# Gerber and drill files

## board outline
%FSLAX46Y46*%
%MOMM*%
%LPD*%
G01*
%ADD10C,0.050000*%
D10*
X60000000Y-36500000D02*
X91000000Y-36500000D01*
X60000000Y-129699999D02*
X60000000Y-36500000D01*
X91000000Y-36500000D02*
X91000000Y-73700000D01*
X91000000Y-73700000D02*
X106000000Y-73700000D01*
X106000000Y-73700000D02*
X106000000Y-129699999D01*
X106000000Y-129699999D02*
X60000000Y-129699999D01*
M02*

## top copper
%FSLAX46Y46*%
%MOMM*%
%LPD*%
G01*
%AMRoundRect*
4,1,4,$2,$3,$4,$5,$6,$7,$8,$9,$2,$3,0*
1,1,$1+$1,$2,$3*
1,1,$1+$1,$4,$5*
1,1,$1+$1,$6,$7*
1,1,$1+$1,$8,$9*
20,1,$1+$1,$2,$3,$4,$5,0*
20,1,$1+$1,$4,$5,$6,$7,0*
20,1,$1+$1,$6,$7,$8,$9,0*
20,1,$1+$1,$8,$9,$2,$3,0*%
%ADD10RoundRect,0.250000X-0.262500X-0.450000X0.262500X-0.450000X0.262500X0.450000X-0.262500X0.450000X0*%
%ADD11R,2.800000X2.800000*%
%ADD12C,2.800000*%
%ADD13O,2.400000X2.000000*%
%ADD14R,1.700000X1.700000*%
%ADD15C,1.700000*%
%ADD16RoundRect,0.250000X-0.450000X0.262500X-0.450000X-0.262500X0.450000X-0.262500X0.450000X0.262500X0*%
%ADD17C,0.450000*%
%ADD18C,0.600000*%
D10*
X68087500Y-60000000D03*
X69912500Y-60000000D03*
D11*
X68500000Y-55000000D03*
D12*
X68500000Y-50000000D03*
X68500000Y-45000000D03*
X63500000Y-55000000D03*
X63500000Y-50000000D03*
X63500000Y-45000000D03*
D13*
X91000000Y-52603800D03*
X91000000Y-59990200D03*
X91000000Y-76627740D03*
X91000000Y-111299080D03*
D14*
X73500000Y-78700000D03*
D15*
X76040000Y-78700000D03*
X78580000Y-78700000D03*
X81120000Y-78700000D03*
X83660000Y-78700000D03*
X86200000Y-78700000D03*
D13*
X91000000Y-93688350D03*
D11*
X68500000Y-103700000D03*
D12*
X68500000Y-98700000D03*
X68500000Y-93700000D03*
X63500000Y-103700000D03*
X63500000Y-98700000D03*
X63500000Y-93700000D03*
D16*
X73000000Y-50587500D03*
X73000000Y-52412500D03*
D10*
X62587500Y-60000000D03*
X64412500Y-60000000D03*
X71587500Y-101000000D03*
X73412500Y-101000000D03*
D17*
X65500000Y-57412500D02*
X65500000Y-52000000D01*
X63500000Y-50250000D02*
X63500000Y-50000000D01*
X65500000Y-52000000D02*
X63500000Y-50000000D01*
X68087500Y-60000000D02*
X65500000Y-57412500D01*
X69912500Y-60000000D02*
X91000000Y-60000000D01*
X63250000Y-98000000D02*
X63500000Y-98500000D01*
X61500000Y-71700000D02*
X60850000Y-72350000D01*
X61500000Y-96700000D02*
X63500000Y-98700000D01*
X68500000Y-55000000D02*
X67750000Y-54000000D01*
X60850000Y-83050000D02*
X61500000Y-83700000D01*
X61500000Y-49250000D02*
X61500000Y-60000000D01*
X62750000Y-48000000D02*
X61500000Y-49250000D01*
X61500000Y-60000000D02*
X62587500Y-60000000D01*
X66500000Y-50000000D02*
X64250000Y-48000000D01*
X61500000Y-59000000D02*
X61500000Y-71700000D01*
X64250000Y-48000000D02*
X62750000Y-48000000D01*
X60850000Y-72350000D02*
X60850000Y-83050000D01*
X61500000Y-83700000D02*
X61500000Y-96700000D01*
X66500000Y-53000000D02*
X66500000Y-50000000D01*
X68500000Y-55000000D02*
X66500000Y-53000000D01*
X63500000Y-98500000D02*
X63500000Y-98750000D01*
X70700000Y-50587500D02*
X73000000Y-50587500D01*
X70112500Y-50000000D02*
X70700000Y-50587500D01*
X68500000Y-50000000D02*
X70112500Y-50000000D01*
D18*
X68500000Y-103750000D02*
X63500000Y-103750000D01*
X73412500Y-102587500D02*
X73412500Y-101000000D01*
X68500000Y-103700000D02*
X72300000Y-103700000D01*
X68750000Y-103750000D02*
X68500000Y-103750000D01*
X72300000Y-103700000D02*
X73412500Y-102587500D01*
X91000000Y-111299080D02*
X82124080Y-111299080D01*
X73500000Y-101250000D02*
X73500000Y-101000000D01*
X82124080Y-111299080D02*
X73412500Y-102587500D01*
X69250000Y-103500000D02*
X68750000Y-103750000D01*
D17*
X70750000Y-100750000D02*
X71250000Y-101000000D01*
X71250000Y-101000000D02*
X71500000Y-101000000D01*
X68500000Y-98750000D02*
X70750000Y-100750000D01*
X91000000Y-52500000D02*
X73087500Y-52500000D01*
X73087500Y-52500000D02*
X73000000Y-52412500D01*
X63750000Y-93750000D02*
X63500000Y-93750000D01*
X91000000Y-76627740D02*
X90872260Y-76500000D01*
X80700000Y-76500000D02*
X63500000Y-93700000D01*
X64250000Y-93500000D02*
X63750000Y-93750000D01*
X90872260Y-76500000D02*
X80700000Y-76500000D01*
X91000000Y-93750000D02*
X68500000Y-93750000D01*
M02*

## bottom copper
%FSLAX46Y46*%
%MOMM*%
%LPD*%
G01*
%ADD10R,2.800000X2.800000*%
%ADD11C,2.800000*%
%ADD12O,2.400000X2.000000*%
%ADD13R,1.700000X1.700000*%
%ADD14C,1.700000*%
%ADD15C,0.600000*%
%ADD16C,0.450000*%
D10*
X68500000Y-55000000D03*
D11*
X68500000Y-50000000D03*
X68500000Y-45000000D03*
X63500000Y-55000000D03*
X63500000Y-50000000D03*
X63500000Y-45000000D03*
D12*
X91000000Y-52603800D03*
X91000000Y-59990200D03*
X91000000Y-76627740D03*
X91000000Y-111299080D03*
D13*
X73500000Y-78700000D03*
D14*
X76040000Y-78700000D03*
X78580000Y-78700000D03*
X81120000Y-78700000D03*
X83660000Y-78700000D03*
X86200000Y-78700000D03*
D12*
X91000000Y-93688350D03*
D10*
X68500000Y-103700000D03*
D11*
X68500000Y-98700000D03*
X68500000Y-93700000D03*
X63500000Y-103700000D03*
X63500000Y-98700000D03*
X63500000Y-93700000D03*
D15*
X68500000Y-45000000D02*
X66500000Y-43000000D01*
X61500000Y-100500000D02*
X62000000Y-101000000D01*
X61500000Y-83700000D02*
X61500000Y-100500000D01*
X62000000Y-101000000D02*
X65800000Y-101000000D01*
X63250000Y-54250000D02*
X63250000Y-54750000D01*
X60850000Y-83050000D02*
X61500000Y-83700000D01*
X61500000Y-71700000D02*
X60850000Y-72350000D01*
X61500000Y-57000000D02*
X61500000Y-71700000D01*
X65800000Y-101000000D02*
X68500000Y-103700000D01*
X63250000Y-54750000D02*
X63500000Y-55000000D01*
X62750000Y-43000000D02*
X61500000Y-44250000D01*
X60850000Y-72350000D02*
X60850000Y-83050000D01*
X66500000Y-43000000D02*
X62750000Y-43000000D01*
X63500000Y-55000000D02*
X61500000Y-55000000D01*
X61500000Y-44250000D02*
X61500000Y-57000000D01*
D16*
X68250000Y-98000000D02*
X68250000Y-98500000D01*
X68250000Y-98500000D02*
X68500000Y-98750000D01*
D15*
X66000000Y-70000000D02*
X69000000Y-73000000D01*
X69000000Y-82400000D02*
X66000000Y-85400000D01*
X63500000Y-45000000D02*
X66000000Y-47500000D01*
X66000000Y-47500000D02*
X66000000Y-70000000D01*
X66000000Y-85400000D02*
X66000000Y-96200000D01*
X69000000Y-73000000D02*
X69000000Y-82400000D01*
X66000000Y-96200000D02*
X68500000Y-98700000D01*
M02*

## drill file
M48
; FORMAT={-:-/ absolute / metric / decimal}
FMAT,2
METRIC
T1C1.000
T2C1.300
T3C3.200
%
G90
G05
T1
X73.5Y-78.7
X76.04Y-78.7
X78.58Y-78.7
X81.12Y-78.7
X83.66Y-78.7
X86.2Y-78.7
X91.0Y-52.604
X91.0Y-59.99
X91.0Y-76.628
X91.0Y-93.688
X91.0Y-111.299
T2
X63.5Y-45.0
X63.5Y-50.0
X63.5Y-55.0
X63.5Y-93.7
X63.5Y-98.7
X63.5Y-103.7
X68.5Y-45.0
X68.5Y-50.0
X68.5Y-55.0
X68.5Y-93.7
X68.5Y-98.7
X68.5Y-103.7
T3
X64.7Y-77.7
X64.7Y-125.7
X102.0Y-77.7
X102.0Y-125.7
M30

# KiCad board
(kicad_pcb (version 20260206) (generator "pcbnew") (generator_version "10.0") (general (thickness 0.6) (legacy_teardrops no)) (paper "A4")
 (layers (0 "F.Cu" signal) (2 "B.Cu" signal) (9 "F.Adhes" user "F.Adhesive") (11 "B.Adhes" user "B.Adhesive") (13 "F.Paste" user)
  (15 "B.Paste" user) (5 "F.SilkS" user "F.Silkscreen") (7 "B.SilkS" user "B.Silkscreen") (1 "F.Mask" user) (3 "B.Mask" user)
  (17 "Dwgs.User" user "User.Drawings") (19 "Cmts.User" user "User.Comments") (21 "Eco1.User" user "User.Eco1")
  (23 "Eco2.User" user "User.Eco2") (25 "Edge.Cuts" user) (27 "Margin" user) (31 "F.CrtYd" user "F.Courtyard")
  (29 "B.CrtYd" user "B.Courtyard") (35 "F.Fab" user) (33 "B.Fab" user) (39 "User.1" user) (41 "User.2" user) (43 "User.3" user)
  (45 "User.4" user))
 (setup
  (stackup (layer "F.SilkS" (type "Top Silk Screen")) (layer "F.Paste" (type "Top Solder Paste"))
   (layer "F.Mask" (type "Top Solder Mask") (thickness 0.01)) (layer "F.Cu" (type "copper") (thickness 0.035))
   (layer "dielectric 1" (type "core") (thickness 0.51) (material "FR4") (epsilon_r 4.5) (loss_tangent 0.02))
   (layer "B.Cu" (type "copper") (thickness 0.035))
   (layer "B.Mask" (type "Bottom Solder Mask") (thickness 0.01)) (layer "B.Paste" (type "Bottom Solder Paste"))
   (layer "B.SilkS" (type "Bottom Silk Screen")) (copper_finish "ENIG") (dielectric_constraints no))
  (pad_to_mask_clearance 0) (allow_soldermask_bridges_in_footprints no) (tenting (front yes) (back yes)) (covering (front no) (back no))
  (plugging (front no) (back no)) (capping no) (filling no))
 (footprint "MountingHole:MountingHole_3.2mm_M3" (layer "F.Cu") (at 64.7 77.7)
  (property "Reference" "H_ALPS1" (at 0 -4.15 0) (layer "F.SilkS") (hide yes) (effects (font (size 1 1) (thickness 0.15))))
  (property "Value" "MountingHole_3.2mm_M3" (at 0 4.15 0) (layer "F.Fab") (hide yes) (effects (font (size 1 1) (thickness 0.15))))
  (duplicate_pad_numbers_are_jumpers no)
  (pad "" np_thru_hole circle (at 0 0) (size 3.2 3.2) (drill 3.2) (layers "*.Cu" "*.Mask")))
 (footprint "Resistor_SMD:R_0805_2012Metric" (layer "F.Cu") (at 69 60)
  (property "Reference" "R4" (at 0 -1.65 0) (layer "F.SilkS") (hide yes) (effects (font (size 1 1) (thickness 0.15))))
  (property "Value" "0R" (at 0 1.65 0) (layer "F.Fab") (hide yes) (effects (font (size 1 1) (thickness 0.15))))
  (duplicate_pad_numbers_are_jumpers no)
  (pad "1" smd roundrect (at -0.9125 0) (size 1.025 1.4) (layers "F.Cu" "F.Mask" "F.Paste") (roundrect_rratio 0.243902) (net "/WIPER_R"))
  (pad "2" smd roundrect (at 0.9125 0) (size 1.025 1.4) (layers "F.Cu" "F.Mask" "F.Paste") (roundrect_rratio 0.243902) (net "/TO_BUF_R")))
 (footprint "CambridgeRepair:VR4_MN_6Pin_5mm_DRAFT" (layer "F.Cu") (at 63.5 50)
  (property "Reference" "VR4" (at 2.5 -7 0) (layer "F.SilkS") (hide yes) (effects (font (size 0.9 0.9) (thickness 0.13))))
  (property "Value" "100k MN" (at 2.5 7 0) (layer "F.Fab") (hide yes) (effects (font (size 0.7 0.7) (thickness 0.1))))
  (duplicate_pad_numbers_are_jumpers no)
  (pad "1" thru_hole rect (at 5 5) (size 2.8 2.8) (drill 1.3) (layers "*.Cu" "*.Mask") (remove_unused_layers no) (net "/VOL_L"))
  (pad "2" thru_hole circle (at 5 0) (size 2.8 2.8) (drill 1.3) (layers "*.Cu" "*.Mask") (remove_unused_layers no) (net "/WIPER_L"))
  (pad "3" thru_hole circle (at 5 -5) (size 2.8 2.8) (drill 1.3) (layers "*.Cu" "*.Mask") (remove_unused_layers no) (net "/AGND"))
  (pad "4" thru_hole circle (at 0 5) (size 2.8 2.8) (drill 1.3) (layers "*.Cu" "*.Mask") (remove_unused_layers no) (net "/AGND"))
  (pad "5" thru_hole circle (at 0 0) (size 2.8 2.8) (drill 1.3) (layers "*.Cu" "*.Mask") (remove_unused_layers no) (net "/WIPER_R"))
  (pad "6" thru_hole circle (at 0 -5) (size 2.8 2.8) (drill 1.3) (layers "*.Cu" "*.Mask") (remove_unused_layers no) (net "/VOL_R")))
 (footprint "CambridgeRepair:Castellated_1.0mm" (layer "F.Cu") (at 91 52.6038)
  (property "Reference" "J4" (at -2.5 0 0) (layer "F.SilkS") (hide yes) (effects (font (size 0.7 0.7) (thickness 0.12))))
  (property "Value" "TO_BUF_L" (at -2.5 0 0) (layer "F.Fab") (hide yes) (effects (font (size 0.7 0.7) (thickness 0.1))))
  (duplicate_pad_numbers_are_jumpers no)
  (pad "1" thru_hole oval (at 0 0) (size 2.4 2) (drill 1) (layers "*.Cu" "*.Mask") (remove_unused_layers no) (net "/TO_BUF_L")
   (solder_mask_margin 0.05)))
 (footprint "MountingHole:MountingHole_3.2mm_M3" (layer "F.Cu") (at 102 77.7)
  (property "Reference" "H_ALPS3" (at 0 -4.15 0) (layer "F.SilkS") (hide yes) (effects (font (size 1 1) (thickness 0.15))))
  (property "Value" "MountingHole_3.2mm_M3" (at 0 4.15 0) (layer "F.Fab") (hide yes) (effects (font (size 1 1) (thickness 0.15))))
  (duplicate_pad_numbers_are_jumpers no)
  (pad "" np_thru_hole circle (at 0 0) (size 3.2 3.2) (drill 3.2) (layers "*.Cu" "*.Mask")))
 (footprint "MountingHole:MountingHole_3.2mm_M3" (layer "F.Cu") (at 102 125.7)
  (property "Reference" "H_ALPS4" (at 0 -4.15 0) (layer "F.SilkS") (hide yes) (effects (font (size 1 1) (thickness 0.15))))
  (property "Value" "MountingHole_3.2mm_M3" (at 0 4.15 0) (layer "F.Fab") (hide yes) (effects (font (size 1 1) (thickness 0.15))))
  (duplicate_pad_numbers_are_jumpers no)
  (pad "" np_thru_hole circle (at 0 0) (size 3.2 3.2) (drill 3.2) (layers "*.Cu" "*.Mask")))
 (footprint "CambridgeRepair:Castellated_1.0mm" (layer "F.Cu") (at 91 59.9902)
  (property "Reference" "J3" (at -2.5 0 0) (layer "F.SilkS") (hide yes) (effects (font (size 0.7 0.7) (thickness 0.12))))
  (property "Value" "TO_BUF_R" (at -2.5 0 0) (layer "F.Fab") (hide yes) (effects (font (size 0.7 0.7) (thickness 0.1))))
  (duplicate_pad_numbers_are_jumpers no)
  (pad "1" thru_hole oval (at 0 0) (size 2.4 2) (drill 1) (layers "*.Cu" "*.Mask") (remove_unused_layers no) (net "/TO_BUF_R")
   (solder_mask_margin 0.05)))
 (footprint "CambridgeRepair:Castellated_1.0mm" (layer "F.Cu") (at 91 76.62774)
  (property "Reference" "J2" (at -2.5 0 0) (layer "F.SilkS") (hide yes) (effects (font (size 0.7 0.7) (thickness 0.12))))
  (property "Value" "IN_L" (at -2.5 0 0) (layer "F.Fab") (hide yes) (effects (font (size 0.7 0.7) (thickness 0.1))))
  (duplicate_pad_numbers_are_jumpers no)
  (pad "1" thru_hole oval (at 0 0) (size 2.4 2) (drill 1) (layers "*.Cu" "*.Mask") (remove_unused_layers no) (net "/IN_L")
   (solder_mask_margin 0.05)))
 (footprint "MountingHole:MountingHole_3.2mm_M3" (layer "F.Cu") (at 64.7 125.7)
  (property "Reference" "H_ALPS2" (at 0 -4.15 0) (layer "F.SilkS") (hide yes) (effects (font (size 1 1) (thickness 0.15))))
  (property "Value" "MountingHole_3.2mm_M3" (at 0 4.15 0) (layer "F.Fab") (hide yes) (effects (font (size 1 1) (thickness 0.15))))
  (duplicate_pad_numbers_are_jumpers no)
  (pad "" np_thru_hole circle (at 0 0) (size 3.2 3.2) (drill 3.2) (layers "*.Cu" "*.Mask")))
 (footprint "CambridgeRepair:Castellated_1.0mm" (layer "F.Cu") (at 91 111.29908)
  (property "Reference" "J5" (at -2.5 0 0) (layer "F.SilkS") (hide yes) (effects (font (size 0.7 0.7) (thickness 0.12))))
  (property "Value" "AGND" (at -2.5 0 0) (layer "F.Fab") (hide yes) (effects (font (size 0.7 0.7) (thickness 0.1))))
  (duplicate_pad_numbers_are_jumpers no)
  (pad "1" thru_hole oval (at 0 0) (size 2.4 2) (drill 1) (layers "*.Cu" "*.Mask") (remove_unused_layers no) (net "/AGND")
   (solder_mask_margin 0.05)))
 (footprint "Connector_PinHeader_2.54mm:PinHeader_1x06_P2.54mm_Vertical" (layer "F.Cu") (at 73.5 78.7 90)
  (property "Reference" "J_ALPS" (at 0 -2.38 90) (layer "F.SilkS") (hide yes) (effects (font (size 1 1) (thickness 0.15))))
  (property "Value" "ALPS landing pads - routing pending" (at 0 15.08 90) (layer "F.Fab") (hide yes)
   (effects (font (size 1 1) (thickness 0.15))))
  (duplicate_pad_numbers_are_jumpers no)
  (pad "1" thru_hole rect (at 0 0 90) (size 1.7 1.7) (drill 1) (layers "*.Cu" "*.Mask") (remove_unused_layers no) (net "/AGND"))
  (pad "2" thru_hole circle (at 0 2.54 90) (size 1.7 1.7) (drill 1) (layers "*.Cu" "*.Mask") (remove_unused_layers no) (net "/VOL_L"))
  (pad "3" thru_hole circle (at 0 5.08 90) (size 1.7 1.7) (drill 1) (layers "*.Cu" "*.Mask") (remove_unused_layers no) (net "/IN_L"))
  (pad "4" thru_hole circle (at 0 7.62 90) (size 1.7 1.7) (drill 1) (layers "*.Cu" "*.Mask") (remove_unused_layers no) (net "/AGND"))
  (pad "5" thru_hole circle (at 0 10.16 90) (size 1.7 1.7) (drill 1) (layers "*.Cu" "*.Mask") (remove_unused_layers no) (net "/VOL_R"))
  (pad "6" thru_hole circle (at 0 12.7 90) (size 1.7 1.7) (drill 1) (layers "*.Cu" "*.Mask") (remove_unused_layers no) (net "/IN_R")))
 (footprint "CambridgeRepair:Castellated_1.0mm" (layer "F.Cu") (at 91 93.68835)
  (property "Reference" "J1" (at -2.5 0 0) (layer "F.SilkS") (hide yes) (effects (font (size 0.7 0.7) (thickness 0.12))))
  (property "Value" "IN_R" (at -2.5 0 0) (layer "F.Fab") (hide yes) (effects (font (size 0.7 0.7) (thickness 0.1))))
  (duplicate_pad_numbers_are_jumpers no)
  (pad "1" thru_hole oval (at 0 0) (size 2.4 2) (drill 1) (layers "*.Cu" "*.Mask") (remove_unused_layers no) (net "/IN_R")
   (solder_mask_margin 0.05)))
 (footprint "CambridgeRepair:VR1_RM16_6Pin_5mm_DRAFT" (layer "F.Cu") (at 63.5 98.7)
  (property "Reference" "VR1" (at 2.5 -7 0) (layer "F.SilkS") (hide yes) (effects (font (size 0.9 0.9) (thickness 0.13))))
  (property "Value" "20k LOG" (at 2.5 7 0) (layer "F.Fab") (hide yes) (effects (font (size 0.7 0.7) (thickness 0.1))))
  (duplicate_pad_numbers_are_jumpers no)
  (pad "1" thru_hole rect (at 5 5) (size 2.8 2.8) (drill 1.3) (layers "*.Cu" "*.Mask") (remove_unused_layers no) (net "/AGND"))
  (pad "2" thru_hole circle (at 5 0) (size 2.8 2.8) (drill 1.3) (layers "*.Cu" "*.Mask") (remove_unused_layers no) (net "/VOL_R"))
  (pad "3" thru_hole circle (at 5 -5) (size 2.8 2.8) (drill 1.3) (layers "*.Cu" "*.Mask") (remove_unused_layers no) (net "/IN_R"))
  (pad "4" thru_hole circle (at 0 5) (size 2.8 2.8) (drill 1.3) (layers "*.Cu" "*.Mask") (remove_unused_layers no) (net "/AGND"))
  (pad "5" thru_hole circle (at 0 0) (size 2.8 2.8) (drill 1.3) (layers "*.Cu" "*.Mask") (remove_unused_layers no) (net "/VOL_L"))
  (pad "6" thru_hole circle (at 0 -5) (size 2.8 2.8) (drill 1.3) (layers "*.Cu" "*.Mask") (remove_unused_layers no) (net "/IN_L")))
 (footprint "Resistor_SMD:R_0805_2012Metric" (layer "F.Cu") (at 73 51.5 -90)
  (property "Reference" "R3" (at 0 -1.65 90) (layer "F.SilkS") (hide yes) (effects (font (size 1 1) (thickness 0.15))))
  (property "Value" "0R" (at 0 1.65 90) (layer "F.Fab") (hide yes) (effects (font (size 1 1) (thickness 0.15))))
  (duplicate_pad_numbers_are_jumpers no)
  (pad "1" smd roundrect (at -0.9125 0 270) (size 1.025 1.4) (layers "F.Cu" "F.Mask" "F.Paste") (roundrect_rratio 0.243902) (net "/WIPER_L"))
  (pad "2" smd roundrect (at 0.9125 0 270) (size 1.025 1.4) (layers "F.Cu" "F.Mask" "F.Paste") (roundrect_rratio 0.243902) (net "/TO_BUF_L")))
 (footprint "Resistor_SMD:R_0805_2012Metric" (layer "F.Cu") (at 63.5 60)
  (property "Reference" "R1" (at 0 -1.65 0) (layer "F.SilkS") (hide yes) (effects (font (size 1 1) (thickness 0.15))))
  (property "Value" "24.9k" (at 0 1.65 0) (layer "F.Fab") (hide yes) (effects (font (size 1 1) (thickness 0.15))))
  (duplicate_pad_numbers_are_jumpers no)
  (pad "1" smd roundrect (at -0.9125 0) (size 1.025 1.4) (layers "F.Cu" "F.Mask" "F.Paste") (roundrect_rratio 0.243902) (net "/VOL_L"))
  (pad "2" smd roundrect (at 0.9125 0) (size 1.025 1.4) (layers "F.Cu" "F.Mask" "F.Paste") (roundrect_rratio 0.243902) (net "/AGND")))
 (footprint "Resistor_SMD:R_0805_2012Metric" (layer "F.Cu") (at 72.5 101)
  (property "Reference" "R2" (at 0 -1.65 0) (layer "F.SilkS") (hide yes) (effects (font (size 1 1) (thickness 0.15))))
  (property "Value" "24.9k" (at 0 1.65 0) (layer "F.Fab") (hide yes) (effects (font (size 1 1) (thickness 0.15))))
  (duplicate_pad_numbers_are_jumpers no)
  (pad "1" smd roundrect (at -0.9125 0) (size 1.025 1.4) (layers "F.Cu" "F.Mask" "F.Paste") (roundrect_rratio 0.243902) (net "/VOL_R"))
  (pad "2" smd roundrect (at 0.9125 0) (size 1.025 1.4) (layers "F.Cu" "F.Mask" "F.Paste") (roundrect_rratio 0.243902) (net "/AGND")))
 (gr_line (start 60 36.5) (end 91 36.5) (stroke (width 0.05) (type default)) (layer "Edge.Cuts"))
 (gr_line (start 60 129.699999) (end 60 36.5) (stroke (width 0.05) (type default)) (layer "Edge.Cuts"))
 (gr_line (start 91 36.5) (end 91 73.7) (stroke (width 0.05) (type default)) (layer "Edge.Cuts"))
 (gr_line (start 91 73.7) (end 106 73.7) (stroke (width 0.05) (type default)) (layer "Edge.Cuts"))
 (gr_line (start 106 73.7) (end 106 129.699999) (stroke (width 0.05) (type default)) (layer "Edge.Cuts"))
 (gr_line (start 106 129.699999) (end 60 129.699999) (stroke (width 0.05) (type default)) (layer "Edge.Cuts"))
 (segment (start 65.5 57.4125) (end 65.5 52) (width 0.45) (layer "F.Cu") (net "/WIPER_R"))
 (segment (start 63.5 50.25) (end 63.5 50) (width 0.45) (layer "F.Cu") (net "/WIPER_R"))
 (segment (start 65.5 52) (end 63.5 50) (width 0.45) (layer "F.Cu") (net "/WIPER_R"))
 (segment (start 68.0875 60) (end 65.5 57.4125) (width 0.45) (layer "F.Cu") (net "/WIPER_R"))
 (segment (start 69.9125 60) (end 91 60) (width 0.45) (layer "F.Cu") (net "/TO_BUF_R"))
 (segment (start 63.25 98) (end 63.5 98.5) (width 0.45) (layer "F.Cu") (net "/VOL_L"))
 (segment (start 61.5 71.7) (end 60.85 72.35) (width 0.45) (layer "F.Cu") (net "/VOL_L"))
 (segment (start 61.5 96.7) (end 63.5 98.7) (width 0.45) (layer "F.Cu") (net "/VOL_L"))
 (segment (start 68.5 55) (end 67.75 54) (width 0.45) (layer "F.Cu") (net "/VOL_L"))
 (segment (start 60.85 83.05) (end 61.5 83.7) (width 0.45) (layer "F.Cu") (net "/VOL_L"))
 (segment (start 61.5 49.25) (end 61.5 60) (width 0.45) (layer "F.Cu") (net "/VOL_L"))
 (segment (start 62.75 48) (end 61.5 49.25) (width 0.45) (layer "F.Cu") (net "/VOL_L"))
 (segment (start 61.5 60) (end 62.5875 60) (width 0.45) (layer "F.Cu") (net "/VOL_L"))
 (segment (start 66.5 50) (end 64.25 48) (width 0.45) (layer "F.Cu") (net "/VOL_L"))
 (segment (start 61.5 59) (end 61.5 71.7) (width 0.45) (layer "F.Cu") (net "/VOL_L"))
 (segment (start 64.25 48) (end 62.75 48) (width 0.45) (layer "F.Cu") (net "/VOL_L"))
 (segment (start 60.85 72.35) (end 60.85 83.05) (width 0.45) (layer "F.Cu") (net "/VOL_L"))
 (segment (start 61.5 83.7) (end 61.5 96.7) (width 0.45) (layer "F.Cu") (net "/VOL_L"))
 (segment (start 66.5 53) (end 66.5 50) (width 0.45) (layer "F.Cu") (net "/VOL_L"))
 (segment (start 68.5 55) (end 66.5 53) (width 0.45) (layer "F.Cu") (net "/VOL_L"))
 (segment (start 63.5 98.5) (end 63.5 98.75) (width 0.45) (layer "F.Cu") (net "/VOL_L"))
 (segment (start 70.7 50.5875) (end 73 50.5875) (width 0.45) (layer "F.Cu") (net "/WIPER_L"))
 (segment (start 70.1125 50) (end 70.7 50.5875) (width 0.45) (layer "F.Cu") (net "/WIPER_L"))
 (segment (start 68.5 50) (end 70.1125 50) (width 0.45) (layer "F.Cu") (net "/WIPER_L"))
 (segment (start 68.5 103.75) (end 63.5 103.75) (width 0.6) (layer "F.Cu") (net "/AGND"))
 (segment (start 73.4125 102.5875) (end 73.4125 101) (width 0.6) (layer "F.Cu") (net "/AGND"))
 (segment (start 68.5 103.7) (end 72.3 103.7) (width 0.6) (layer "F.Cu") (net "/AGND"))
 (segment (start 68.75 103.75) (end 68.5 103.75) (width 0.6) (layer "F.Cu") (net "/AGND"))
 (segment (start 72.3 103.7) (end 73.4125 102.5875) (width 0.6) (layer "F.Cu") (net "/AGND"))
 (segment (start 91 111.29908) (end 82.12408 111.29908) (width 0.6) (layer "F.Cu") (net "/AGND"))
 (segment (start 73.5 101.25) (end 73.5 101) (width 0.6) (layer "F.Cu") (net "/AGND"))
 (segment (start 82.12408 111.29908) (end 73.4125 102.5875) (width 0.6) (layer "F.Cu") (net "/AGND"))
 (segment (start 69.25 103.5) (end 68.75 103.75) (width 0.6) (layer "F.Cu") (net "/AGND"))
 (segment (start 68.5 45) (end 66.5 43) (width 0.6) (layer "B.Cu") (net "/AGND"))
 (segment (start 61.5 100.5) (end 62 101) (width 0.6) (layer "B.Cu") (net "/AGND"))
 (segment (start 61.5 83.7) (end 61.5 100.5) (width 0.6) (layer "B.Cu") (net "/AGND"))
 (segment (start 62 101) (end 65.8 101) (width 0.6) (layer "B.Cu") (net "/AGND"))
 (segment (start 63.25 54.25) (end 63.25 54.75) (width 0.6) (layer "B.Cu") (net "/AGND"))
 (segment (start 60.85 83.05) (end 61.5 83.7) (width 0.6) (layer "B.Cu") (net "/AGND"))
 (segment (start 61.5 71.7) (end 60.85 72.35) (width 0.6) (layer "B.Cu") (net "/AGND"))
 (segment (start 61.5 57) (end 61.5 71.7) (width 0.6) (layer "B.Cu") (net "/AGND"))
 (segment (start 65.8 101) (end 68.5 103.7) (width 0.6) (layer "B.Cu") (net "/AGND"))
 (segment (start 63.25 54.75) (end 63.5 55) (width 0.6) (layer "B.Cu") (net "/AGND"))
 (segment (start 62.75 43) (end 61.5 44.25) (width 0.6) (layer "B.Cu") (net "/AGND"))
 (segment (start 60.85 72.35) (end 60.85 83.05) (width 0.6) (layer "B.Cu") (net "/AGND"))
 (segment (start 66.5 43) (end 62.75 43) (width 0.6) (layer "B.Cu") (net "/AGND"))
 (segment (start 63.5 55) (end 61.5 55) (width 0.6) (layer "B.Cu") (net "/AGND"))
 (segment (start 61.5 44.25) (end 61.5 57) (width 0.6) (layer "B.Cu") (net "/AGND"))
 (segment (start 70.75 100.75) (end 71.25 101) (width 0.45) (layer "F.Cu") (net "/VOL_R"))
 (segment (start 71.25 101) (end 71.5 101) (width 0.45) (layer "F.Cu") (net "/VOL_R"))
 (segment (start 68.5 98.75) (end 70.75 100.75) (width 0.45) (layer "F.Cu") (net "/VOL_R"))
 (segment (start 68.25 98) (end 68.25 98.5) (width 0.45) (layer "B.Cu") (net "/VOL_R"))
 (segment (start 68.25 98.5) (end 68.5 98.75) (width 0.45) (layer "B.Cu") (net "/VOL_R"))
 (segment (start 66 70) (end 69 73) (width 0.6) (layer "B.Cu") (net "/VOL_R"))
 (segment (start 69 82.4) (end 66 85.4) (width 0.6) (layer "B.Cu") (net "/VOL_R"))
 (segment (start 63.5 45) (end 66 47.5) (width 0.6) (layer "B.Cu") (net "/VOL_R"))
 (segment (start 66 47.5) (end 66 70) (width 0.6) (layer "B.Cu") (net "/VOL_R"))
 (segment (start 66 85.4) (end 66 96.2) (width 0.6) (layer "B.Cu") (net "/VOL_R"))
 (segment (start 69 73) (end 69 82.4) (width 0.6) (layer "B.Cu") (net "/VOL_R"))
 (segment (start 66 96.2) (end 68.5 98.7) (width 0.6) (layer "B.Cu") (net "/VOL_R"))
 (segment (start 91 52.5) (end 73.0875 52.5) (width 0.45) (layer "F.Cu") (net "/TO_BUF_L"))
 (segment (start 73.0875 52.5) (end 73 52.4125) (width 0.45) (layer "F.Cu") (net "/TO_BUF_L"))
 (segment (start 63.75 93.75) (end 63.5 93.75) (width 0.45) (layer "F.Cu") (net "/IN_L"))
 (segment (start 91 76.62774) (end 90.87226 76.5) (width 0.45) (layer "F.Cu") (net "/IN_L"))
 (segment (start 80.7 76.5) (end 63.5 93.7) (width 0.45) (layer "F.Cu") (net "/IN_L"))
 (segment (start 64.25 93.5) (end 63.75 93.75) (width 0.45) (layer "F.Cu") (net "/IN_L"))
 (segment (start 90.87226 76.5) (end 80.7 76.5) (width 0.45) (layer "F.Cu") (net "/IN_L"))
 (segment (start 91 93.75) (end 68.5 93.75) (width 0.45) (layer "F.Cu") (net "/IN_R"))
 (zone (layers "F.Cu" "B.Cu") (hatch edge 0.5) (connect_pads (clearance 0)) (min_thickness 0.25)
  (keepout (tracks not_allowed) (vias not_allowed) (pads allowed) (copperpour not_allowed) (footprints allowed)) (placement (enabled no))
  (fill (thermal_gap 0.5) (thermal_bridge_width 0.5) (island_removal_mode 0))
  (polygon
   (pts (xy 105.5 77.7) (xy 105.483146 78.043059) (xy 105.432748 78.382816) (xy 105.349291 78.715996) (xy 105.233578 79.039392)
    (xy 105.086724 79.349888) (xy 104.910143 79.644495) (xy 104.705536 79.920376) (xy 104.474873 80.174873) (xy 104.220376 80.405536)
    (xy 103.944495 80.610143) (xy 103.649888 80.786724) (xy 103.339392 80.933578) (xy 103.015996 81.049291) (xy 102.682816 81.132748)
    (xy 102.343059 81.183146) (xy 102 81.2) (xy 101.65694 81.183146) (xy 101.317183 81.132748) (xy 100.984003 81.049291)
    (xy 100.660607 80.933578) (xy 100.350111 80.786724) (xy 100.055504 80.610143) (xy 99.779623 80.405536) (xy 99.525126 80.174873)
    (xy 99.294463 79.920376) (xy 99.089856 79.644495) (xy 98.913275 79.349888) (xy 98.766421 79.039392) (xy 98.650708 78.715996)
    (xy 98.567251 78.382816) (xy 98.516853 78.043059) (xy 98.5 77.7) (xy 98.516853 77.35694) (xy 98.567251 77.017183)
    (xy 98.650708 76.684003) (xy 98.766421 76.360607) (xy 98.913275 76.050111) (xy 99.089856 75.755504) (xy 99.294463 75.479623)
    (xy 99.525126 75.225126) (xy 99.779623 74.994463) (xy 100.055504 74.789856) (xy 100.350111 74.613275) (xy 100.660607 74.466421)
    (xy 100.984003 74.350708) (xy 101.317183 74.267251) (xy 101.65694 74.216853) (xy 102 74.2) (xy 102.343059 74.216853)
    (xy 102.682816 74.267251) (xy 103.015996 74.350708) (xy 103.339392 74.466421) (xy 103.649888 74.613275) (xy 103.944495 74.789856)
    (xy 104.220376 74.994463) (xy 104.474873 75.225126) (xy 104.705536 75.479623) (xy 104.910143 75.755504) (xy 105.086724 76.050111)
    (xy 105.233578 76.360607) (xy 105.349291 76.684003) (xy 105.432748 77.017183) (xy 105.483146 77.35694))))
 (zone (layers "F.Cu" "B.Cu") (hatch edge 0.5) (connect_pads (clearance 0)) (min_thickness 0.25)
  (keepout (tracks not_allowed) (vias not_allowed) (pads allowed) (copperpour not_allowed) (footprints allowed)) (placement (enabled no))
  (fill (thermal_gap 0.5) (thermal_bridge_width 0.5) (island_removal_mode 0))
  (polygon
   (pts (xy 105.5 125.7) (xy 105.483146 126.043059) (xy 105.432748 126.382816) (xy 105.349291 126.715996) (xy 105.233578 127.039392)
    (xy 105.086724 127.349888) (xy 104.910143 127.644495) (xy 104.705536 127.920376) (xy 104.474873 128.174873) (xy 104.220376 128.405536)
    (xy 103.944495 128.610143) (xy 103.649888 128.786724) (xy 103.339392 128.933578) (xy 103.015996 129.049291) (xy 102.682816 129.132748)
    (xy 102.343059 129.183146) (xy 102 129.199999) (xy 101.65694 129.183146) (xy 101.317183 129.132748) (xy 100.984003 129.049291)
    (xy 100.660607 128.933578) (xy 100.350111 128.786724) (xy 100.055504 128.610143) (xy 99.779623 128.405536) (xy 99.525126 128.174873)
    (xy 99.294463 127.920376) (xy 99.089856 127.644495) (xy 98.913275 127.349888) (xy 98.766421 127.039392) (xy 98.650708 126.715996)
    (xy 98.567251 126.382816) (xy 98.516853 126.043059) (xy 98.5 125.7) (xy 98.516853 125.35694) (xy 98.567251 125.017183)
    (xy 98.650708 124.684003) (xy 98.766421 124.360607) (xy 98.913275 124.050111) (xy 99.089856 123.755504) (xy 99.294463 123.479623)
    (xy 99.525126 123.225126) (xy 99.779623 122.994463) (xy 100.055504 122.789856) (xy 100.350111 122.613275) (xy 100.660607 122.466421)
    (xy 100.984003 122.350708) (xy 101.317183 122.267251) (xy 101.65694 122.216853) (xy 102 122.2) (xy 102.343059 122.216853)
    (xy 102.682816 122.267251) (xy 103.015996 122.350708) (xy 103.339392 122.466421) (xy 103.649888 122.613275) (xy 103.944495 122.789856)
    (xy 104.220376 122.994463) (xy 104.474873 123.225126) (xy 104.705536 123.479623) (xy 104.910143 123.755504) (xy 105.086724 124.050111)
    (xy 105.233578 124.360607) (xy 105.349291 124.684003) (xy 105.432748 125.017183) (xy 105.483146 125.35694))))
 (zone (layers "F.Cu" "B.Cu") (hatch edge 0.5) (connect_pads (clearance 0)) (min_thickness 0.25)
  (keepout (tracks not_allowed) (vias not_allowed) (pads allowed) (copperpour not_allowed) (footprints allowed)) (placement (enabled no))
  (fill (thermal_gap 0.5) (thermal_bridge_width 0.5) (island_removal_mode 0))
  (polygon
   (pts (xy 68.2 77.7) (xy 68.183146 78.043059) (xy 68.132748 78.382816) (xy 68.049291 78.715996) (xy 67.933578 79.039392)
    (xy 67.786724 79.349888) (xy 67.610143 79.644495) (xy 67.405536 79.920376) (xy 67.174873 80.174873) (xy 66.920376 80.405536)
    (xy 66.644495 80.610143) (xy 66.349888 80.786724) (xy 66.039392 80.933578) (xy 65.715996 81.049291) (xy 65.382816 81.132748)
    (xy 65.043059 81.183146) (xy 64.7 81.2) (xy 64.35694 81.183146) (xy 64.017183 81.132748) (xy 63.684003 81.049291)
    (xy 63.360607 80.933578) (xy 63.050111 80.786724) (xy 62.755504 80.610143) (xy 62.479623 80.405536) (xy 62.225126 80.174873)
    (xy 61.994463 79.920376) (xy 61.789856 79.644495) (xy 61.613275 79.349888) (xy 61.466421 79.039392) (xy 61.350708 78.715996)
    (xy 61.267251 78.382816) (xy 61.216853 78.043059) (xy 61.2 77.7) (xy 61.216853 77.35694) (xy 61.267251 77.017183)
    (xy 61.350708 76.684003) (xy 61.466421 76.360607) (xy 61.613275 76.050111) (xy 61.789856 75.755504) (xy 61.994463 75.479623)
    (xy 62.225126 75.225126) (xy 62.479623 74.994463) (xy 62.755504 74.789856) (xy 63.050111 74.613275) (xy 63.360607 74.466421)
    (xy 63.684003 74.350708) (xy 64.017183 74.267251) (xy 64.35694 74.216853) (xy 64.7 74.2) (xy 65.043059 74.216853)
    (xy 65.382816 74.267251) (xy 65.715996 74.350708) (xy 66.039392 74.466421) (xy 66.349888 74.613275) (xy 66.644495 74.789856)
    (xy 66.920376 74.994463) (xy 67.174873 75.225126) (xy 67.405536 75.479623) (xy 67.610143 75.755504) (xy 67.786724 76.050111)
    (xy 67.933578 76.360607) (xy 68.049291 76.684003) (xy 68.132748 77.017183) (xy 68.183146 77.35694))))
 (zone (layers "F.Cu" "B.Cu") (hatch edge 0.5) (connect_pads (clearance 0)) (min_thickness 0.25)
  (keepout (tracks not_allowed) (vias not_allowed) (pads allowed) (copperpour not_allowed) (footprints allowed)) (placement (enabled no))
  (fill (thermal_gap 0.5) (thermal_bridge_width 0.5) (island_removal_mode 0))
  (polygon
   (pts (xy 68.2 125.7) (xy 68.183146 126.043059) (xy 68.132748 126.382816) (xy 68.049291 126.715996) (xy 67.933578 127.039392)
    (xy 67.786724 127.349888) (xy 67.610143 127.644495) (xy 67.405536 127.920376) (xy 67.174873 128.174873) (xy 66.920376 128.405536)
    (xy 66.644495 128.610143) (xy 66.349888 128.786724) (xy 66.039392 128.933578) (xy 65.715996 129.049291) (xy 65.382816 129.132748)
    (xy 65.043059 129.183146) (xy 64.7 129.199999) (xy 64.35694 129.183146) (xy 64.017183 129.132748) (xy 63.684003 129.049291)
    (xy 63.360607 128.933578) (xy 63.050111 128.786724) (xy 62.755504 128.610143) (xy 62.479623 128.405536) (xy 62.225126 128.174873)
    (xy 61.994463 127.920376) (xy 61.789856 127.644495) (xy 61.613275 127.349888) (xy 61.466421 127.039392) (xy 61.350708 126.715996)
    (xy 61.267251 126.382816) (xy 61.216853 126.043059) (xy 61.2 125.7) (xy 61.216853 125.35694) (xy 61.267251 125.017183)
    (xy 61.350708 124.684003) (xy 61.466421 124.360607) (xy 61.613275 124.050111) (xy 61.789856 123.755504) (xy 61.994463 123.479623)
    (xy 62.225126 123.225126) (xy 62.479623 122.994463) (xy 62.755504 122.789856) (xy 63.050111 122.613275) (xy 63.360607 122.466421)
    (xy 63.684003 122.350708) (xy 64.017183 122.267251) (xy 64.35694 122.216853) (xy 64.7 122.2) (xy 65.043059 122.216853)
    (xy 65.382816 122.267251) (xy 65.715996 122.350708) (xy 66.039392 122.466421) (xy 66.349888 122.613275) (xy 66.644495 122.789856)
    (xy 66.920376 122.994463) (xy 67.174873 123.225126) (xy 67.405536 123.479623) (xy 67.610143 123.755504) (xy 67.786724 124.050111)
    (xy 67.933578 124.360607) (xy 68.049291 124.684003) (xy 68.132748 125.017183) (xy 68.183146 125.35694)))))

